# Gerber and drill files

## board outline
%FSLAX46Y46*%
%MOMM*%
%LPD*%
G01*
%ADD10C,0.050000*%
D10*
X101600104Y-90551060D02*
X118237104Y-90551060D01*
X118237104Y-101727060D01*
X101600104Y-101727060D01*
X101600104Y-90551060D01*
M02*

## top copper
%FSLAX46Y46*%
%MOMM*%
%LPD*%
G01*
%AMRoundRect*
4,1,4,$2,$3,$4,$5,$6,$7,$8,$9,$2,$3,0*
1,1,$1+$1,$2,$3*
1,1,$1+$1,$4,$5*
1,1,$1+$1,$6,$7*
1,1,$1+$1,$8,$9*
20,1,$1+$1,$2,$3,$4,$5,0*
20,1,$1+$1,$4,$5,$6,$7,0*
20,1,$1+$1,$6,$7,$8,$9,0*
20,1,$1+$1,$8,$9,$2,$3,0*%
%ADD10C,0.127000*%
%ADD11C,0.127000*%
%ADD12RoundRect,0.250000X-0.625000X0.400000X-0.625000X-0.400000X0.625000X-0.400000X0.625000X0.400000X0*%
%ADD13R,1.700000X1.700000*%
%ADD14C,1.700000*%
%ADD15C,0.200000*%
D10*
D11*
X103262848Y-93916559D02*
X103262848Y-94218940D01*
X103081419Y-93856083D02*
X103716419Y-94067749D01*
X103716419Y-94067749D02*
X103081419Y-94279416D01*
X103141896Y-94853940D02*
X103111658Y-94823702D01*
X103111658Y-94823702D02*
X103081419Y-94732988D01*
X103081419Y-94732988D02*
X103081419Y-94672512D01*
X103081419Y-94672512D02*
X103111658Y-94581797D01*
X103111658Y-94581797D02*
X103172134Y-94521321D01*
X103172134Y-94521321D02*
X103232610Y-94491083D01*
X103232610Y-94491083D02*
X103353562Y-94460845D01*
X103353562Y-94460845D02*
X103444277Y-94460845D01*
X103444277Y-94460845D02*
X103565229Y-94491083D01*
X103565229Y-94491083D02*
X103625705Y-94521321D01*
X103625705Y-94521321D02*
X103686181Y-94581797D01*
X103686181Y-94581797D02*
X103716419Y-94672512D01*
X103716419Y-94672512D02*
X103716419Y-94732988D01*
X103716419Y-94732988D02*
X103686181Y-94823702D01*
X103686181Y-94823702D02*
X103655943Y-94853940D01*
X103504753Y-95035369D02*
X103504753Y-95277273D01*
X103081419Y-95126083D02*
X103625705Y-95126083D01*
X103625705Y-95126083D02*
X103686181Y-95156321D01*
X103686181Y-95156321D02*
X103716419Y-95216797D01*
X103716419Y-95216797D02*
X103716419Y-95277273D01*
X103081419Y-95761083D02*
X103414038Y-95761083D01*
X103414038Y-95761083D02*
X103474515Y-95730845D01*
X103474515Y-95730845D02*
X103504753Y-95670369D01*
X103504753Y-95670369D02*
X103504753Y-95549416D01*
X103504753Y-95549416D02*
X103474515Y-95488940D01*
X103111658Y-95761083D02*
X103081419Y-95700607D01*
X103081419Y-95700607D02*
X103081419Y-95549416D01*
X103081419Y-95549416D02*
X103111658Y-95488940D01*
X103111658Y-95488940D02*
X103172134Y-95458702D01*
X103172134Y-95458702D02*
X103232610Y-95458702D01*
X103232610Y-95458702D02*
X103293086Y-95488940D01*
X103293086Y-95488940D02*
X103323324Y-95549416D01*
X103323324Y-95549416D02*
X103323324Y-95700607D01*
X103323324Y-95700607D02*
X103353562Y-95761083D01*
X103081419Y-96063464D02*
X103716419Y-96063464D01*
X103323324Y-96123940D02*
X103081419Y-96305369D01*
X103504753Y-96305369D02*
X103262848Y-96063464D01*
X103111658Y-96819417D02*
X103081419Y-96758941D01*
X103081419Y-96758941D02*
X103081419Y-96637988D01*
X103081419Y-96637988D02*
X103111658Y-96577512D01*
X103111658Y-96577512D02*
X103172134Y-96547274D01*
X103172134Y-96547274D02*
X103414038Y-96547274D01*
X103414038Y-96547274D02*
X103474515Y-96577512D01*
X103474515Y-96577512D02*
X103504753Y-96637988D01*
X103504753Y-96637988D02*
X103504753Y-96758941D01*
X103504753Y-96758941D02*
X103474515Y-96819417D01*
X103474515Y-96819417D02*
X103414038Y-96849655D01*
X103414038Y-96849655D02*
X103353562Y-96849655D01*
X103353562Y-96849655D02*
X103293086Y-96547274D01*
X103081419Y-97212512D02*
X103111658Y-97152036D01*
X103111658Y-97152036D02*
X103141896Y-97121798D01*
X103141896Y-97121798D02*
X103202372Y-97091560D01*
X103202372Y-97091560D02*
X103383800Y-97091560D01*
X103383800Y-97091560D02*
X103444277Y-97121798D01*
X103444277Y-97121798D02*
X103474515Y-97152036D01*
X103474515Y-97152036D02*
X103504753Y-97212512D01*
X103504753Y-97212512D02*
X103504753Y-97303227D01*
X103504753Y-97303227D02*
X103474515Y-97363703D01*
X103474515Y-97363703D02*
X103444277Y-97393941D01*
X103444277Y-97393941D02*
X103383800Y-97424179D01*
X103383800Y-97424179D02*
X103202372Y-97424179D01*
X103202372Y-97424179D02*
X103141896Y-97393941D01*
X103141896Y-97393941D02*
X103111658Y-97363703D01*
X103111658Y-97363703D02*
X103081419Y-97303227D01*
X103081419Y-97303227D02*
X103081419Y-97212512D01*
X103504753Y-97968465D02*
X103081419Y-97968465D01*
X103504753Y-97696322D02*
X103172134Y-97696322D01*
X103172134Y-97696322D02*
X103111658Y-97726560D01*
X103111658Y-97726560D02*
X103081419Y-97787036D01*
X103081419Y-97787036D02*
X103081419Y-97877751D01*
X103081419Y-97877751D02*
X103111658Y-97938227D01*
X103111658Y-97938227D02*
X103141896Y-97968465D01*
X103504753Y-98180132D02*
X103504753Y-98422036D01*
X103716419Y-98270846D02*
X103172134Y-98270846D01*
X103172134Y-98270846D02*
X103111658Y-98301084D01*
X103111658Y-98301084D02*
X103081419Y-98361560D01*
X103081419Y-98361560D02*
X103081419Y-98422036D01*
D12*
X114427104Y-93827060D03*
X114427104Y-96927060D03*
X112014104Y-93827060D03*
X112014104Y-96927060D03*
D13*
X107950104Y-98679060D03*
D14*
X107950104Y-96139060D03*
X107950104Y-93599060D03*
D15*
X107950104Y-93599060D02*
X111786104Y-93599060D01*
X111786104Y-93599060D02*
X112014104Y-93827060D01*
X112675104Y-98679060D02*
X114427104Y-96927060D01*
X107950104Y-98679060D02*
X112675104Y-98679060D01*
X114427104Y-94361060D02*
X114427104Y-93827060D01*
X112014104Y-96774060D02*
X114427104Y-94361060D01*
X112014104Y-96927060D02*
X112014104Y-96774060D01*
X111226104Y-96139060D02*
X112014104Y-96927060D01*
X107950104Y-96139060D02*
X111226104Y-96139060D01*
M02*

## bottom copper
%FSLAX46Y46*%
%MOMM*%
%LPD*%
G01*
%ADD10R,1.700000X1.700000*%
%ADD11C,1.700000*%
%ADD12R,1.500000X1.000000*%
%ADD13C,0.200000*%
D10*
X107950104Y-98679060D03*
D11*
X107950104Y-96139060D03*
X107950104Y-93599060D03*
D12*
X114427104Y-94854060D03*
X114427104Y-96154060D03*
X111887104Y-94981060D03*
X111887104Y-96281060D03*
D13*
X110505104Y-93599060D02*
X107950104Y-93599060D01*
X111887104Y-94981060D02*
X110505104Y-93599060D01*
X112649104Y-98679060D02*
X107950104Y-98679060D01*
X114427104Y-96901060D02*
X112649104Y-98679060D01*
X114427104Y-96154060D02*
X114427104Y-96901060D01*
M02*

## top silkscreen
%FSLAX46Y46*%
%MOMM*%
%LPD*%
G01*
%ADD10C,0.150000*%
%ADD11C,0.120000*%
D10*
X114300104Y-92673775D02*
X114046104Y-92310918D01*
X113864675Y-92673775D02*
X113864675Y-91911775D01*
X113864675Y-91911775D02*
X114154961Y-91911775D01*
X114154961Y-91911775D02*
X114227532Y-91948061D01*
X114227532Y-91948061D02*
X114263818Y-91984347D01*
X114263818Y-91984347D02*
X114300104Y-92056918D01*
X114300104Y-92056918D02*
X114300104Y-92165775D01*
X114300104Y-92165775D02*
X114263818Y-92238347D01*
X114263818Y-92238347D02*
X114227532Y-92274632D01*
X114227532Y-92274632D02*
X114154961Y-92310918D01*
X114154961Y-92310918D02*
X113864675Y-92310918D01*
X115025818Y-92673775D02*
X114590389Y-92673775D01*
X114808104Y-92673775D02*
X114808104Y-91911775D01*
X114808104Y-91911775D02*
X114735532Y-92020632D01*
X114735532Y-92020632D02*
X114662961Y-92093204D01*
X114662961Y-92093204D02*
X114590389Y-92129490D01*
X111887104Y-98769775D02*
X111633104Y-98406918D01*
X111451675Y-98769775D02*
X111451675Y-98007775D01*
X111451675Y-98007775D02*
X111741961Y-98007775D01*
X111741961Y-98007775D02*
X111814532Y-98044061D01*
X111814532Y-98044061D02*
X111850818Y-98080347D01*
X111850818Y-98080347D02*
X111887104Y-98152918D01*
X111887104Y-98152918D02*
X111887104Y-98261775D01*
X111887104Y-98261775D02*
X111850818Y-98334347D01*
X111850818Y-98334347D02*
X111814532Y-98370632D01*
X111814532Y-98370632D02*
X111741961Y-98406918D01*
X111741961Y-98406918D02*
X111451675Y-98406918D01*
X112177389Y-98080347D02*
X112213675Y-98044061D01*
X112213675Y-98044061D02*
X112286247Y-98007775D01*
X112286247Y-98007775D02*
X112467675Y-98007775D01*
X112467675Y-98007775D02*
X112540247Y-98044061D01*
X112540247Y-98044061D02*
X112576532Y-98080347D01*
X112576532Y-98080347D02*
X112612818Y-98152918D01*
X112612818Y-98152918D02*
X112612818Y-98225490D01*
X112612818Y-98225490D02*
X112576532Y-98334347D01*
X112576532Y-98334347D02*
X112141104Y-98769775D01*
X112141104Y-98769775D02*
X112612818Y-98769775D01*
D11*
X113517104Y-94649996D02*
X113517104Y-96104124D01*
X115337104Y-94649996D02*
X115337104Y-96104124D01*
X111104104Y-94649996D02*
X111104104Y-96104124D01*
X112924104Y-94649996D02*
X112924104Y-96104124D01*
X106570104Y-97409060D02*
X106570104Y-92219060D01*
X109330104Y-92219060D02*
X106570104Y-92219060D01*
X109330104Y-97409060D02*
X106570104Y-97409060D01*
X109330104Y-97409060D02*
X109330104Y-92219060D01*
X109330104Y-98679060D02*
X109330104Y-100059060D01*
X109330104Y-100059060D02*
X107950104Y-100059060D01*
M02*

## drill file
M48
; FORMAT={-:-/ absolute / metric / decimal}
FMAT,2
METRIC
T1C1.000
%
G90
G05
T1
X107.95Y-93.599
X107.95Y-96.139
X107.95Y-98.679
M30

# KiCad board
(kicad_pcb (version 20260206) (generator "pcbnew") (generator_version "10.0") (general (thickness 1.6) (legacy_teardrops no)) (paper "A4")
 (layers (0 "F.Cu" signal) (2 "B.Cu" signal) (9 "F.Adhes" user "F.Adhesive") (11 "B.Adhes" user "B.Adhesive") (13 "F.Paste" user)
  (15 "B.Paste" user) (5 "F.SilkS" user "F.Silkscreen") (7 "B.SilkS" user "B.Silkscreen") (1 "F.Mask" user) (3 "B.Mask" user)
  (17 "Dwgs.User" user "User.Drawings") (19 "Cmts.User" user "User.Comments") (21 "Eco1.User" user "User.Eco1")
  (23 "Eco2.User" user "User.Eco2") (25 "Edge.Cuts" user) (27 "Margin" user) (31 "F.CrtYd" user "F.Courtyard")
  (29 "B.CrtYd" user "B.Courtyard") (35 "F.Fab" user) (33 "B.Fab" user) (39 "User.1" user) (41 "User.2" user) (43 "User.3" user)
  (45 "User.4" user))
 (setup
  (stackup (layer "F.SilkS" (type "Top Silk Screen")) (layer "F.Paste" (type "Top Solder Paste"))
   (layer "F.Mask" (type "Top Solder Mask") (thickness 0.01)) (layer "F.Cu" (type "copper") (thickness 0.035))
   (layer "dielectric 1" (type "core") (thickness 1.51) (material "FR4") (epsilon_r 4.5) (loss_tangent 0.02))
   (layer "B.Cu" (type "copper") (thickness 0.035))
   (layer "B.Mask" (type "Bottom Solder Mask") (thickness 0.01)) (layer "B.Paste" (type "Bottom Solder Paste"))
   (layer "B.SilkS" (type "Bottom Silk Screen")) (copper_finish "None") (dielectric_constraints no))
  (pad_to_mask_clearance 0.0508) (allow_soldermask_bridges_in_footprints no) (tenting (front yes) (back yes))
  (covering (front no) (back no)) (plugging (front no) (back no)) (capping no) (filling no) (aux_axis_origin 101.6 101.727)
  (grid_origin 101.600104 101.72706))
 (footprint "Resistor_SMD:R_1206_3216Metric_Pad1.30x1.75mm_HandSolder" (layer "F.Cu") (at 114.427104 95.37706 -90)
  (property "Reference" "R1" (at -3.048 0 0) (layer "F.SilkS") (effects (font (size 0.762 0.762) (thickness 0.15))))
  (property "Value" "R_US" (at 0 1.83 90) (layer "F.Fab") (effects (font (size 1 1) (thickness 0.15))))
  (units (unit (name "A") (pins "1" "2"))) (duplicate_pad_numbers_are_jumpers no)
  (fp_line (start -0.727064 0.91) (end 0.727064 0.91) (stroke (width 0.12) (type solid)) (layer "F.SilkS"))
  (fp_line (start -0.727064 -0.91) (end 0.727064 -0.91) (stroke (width 0.12) (type solid)) (layer "F.SilkS"))
  (pad "1" smd roundrect (at -1.55 0 270) (size 1.3 1.75) (layers "F.Cu" "F.Mask" "F.Paste") (roundrect_rratio 0.192308)
   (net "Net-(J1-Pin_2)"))
  (pad "2" smd roundrect (at 1.55 0 270) (size 1.3 1.75) (layers "F.Cu" "F.Mask" "F.Paste") (roundrect_rratio 0.192308)
   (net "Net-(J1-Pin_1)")))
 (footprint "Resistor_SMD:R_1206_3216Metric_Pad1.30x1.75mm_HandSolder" (layer "F.Cu") (at 112.014104 95.37706 -90)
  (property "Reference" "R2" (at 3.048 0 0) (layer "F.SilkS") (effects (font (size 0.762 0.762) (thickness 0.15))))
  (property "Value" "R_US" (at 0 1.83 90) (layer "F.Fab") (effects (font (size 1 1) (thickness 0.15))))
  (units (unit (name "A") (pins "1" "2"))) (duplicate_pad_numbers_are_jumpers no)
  (fp_line (start -0.727064 0.91) (end 0.727064 0.91) (stroke (width 0.12) (type solid)) (layer "F.SilkS"))
  (fp_line (start -0.727064 -0.91) (end 0.727064 -0.91) (stroke (width 0.12) (type solid)) (layer "F.SilkS"))
  (pad "1" smd roundrect (at -1.55 0 270) (size 1.3 1.75) (layers "F.Cu" "F.Mask" "F.Paste") (roundrect_rratio 0.192308)
   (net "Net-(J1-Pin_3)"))
  (pad "2" smd roundrect (at 1.55 0 270) (size 1.3 1.75) (layers "F.Cu" "F.Mask" "F.Paste") (roundrect_rratio 0.192308)
   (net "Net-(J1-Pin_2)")))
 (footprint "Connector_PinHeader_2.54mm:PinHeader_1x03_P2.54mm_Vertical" (layer "F.Cu") (at 107.950104 98.67906 180)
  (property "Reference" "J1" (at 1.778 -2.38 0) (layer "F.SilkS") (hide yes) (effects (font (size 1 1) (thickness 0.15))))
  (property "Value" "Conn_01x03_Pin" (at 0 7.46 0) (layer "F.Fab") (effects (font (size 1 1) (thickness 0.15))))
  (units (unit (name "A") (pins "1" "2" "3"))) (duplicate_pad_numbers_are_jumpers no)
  (fp_line (start 1.38 1.27) (end 1.38 6.46) (stroke (width 0.12) (type solid)) (layer "F.SilkS"))
  (fp_line (start -1.38 6.46) (end 1.38 6.46) (stroke (width 0.12) (type solid)) (layer "F.SilkS"))
  (fp_line (start -1.38 1.27) (end 1.38 1.27) (stroke (width 0.12) (type solid)) (layer "F.SilkS"))
  (fp_line (start -1.38 1.27) (end -1.38 6.46) (stroke (width 0.12) (type solid)) (layer "F.SilkS"))
  (fp_line (start -1.38 0) (end -1.38 -1.38) (stroke (width 0.12) (type solid)) (layer "F.SilkS"))
  (fp_line (start -1.38 -1.38) (end 0 -1.38) (stroke (width 0.12) (type solid)) (layer "F.SilkS"))
  (pad "1" thru_hole rect (at 0 0 180) (size 1.7 1.7) (drill 1) (layers "*.Cu" "*.Mask") (remove_unused_layers no) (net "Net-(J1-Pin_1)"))
  (pad "2" thru_hole circle (at 0 2.54 180) (size 1.7 1.7) (drill 1) (layers "*.Cu" "*.Mask") (remove_unused_layers no)
   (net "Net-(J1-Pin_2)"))
  (pad "3" thru_hole circle (at 0 5.08 180) (size 1.7 1.7) (drill 1) (layers "*.Cu" "*.Mask") (remove_unused_layers no)
   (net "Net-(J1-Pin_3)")))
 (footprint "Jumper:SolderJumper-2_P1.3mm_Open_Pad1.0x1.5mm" (layer "B.Cu") (at 114.427104 95.50406 -90)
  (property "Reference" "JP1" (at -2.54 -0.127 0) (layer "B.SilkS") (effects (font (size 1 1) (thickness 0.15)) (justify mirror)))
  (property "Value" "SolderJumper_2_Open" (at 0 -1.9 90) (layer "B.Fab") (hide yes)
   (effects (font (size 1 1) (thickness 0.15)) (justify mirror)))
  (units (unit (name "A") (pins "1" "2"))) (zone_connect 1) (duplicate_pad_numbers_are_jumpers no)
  (pad "1" smd rect (at -0.65 0 270) (size 1 1.5) (layers "B.Cu" "B.Mask") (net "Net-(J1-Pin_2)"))
  (pad "2" smd rect (at 0.65 0 270) (size 1 1.5) (layers "B.Cu" "B.Mask") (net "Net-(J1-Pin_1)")))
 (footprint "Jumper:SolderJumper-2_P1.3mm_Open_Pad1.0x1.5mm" (layer "B.Cu") (at 111.887104 95.63106 -90)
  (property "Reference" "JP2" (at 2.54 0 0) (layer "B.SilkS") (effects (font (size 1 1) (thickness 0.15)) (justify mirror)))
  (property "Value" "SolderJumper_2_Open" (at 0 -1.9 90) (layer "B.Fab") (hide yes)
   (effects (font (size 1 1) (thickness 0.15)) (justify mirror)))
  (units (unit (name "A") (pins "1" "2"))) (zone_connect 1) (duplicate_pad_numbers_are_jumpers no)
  (pad "1" smd rect (at -0.65 0 270) (size 1 1.5) (layers "B.Cu" "B.Mask") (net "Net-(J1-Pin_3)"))
  (pad "2" smd rect (at 0.65 0 270) (size 1 1.5) (layers "B.Cu" "B.Mask") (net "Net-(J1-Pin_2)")))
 (gr_rect (start 101.600104 90.55106) (end 118.237104 101.72706) (stroke (width 0.05) (type solid)) (fill no) (layer "Edge.Cuts"))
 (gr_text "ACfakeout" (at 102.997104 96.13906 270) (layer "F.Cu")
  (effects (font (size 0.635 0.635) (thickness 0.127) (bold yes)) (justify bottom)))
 (segment (start 107.950104 93.59906) (end 111.786104 93.59906) (width 0.2) (layer "F.Cu") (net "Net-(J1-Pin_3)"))
 (segment (start 111.786104 93.59906) (end 112.014104 93.82706) (width 0.2) (layer "F.Cu") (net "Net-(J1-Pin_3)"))
 (segment (start 110.505104 93.59906) (end 107.950104 93.59906) (width 0.2) (layer "B.Cu") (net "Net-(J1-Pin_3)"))
 (segment (start 111.887104 94.98106) (end 110.505104 93.59906) (width 0.2) (layer "B.Cu") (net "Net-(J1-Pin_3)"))
 (segment (start 112.675104 98.67906) (end 114.427104 96.92706) (width 0.2) (layer "F.Cu") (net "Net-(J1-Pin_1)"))
 (segment (start 107.950104 98.67906) (end 112.675104 98.67906) (width 0.2) (layer "F.Cu") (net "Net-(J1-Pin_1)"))
 (segment (start 112.649104 98.67906) (end 107.950104 98.67906) (width 0.2) (layer "B.Cu") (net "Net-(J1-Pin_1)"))
 (segment (start 114.427104 96.90106) (end 112.649104 98.67906) (width 0.2) (layer "B.Cu") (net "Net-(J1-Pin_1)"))
 (segment (start 114.427104 96.15406) (end 114.427104 96.90106) (width 0.2) (layer "B.Cu") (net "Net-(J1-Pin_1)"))
 (segment (start 114.427104 94.36106) (end 114.427104 93.82706) (width 0.2) (layer "F.Cu") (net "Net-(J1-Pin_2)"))
 (segment (start 112.014104 96.77406) (end 114.427104 94.36106) (width 0.2) (layer "F.Cu") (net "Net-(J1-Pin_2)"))
 (segment (start 112.014104 96.92706) (end 112.014104 96.77406) (width 0.2) (layer "F.Cu") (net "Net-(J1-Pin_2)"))
 (segment (start 111.226104 96.13906) (end 112.014104 96.92706) (width 0.2) (layer "F.Cu") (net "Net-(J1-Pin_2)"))
 (segment (start 107.950104 96.13906) (end 111.226104 96.13906) (width 0.2) (layer "F.Cu") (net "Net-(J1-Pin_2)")))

